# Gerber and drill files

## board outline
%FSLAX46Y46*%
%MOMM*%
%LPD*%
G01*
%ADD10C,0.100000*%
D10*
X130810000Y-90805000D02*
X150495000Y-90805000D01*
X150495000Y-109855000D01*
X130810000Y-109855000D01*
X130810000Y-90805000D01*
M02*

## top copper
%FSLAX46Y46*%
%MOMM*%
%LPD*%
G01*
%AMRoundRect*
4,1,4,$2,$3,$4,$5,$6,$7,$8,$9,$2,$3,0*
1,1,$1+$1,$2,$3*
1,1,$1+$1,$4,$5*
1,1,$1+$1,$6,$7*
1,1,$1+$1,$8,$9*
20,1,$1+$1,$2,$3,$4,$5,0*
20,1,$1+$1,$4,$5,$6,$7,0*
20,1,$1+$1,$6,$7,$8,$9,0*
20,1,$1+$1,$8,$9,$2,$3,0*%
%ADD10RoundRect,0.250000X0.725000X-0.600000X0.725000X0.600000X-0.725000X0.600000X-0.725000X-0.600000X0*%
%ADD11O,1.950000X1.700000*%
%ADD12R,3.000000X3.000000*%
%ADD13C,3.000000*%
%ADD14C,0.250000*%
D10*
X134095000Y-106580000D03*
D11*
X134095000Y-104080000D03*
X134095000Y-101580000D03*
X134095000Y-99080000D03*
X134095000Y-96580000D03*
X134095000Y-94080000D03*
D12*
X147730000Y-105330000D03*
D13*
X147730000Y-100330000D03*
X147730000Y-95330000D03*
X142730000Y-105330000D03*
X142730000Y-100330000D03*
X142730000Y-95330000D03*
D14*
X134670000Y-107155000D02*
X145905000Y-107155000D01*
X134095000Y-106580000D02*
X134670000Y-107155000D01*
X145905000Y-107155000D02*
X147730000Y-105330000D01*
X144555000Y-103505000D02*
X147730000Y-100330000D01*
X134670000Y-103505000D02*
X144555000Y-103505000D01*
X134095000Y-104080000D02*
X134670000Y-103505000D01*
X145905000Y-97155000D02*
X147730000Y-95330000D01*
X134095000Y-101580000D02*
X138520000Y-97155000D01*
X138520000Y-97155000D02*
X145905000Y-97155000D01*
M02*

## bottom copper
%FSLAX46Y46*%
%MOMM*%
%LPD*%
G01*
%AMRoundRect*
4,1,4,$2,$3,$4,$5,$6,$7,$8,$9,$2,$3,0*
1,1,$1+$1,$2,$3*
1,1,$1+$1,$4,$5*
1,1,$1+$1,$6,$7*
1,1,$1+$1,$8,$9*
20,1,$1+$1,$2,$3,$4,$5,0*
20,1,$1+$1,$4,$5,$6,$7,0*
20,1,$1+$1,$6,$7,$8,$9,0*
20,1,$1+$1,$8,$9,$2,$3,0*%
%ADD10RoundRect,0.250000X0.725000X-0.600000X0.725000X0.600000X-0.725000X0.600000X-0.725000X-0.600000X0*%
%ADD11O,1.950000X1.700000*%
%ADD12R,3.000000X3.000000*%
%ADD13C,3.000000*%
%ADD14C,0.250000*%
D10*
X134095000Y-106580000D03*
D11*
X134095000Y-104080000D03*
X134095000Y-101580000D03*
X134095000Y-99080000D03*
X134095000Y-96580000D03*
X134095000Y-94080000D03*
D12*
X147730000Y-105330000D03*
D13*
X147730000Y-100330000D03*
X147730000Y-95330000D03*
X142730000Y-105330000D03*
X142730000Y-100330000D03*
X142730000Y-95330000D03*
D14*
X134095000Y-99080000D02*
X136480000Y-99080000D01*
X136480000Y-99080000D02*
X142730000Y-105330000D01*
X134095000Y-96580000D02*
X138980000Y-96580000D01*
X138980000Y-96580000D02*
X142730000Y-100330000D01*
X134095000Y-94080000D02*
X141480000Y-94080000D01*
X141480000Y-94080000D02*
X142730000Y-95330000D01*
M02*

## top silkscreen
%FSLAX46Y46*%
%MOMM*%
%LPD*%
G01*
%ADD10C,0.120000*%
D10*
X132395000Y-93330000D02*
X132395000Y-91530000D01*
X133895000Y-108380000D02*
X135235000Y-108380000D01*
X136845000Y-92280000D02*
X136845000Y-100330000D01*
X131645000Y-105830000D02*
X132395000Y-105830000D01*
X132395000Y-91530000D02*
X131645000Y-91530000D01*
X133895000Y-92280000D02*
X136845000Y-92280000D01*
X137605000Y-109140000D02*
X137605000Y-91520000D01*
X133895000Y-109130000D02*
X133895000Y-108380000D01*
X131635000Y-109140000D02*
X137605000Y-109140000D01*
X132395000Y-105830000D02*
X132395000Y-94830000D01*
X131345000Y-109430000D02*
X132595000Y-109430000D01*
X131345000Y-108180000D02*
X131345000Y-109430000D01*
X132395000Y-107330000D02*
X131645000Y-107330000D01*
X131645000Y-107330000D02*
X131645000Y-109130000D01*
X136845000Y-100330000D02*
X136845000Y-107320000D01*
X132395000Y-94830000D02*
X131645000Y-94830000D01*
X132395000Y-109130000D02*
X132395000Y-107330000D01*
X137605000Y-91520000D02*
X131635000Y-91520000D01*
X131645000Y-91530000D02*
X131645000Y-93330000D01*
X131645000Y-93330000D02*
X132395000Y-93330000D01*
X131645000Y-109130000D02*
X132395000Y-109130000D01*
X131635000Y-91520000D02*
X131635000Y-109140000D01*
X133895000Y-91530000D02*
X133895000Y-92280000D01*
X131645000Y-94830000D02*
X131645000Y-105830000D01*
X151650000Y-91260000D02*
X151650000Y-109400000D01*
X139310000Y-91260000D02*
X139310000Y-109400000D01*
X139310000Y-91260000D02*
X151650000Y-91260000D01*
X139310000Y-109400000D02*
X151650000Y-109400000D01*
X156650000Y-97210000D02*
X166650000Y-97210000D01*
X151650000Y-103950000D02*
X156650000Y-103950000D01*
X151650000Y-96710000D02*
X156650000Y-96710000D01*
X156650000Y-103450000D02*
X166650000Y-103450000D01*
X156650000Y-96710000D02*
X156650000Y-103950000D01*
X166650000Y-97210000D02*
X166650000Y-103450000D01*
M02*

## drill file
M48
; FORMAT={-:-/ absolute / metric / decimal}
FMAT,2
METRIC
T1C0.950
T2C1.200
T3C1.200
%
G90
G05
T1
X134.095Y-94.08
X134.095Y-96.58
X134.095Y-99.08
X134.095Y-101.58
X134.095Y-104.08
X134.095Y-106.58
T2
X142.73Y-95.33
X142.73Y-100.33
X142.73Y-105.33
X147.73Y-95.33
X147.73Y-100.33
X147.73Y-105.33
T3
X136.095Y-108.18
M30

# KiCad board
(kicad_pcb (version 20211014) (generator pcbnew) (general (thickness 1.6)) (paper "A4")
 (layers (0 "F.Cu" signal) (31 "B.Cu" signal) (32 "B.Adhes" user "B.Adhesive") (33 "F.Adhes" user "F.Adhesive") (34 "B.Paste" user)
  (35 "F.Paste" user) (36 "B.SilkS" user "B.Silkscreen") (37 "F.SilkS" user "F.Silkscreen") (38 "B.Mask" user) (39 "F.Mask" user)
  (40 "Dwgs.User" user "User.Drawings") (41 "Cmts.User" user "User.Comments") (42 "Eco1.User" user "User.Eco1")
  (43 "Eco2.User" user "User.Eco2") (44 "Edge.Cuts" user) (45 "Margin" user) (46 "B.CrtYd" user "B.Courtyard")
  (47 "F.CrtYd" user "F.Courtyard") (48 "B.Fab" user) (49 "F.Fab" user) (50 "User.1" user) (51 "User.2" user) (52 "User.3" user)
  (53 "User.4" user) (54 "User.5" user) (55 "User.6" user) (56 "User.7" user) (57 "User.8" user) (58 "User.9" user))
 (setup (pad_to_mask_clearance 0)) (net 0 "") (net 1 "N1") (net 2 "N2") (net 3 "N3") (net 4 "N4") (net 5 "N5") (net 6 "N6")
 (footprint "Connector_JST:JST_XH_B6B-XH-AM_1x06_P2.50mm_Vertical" (layer "F.Cu") (at 134.095 106.58 90)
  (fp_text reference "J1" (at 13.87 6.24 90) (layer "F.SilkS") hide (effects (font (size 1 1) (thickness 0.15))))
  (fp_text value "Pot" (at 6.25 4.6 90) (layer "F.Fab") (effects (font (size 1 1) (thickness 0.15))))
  (fp_line (start 13.25 -1.7) (end 15.05 -1.7) (layer "F.SilkS") (width 0.12))
  (fp_line (start -1.8 -0.2) (end -1.8 1.14) (layer "F.SilkS") (width 0.12))
  (fp_line (start 14.3 2.75) (end 6.25 2.75) (layer "F.SilkS") (width 0.12))
  (fp_line (start 0.75 -2.45) (end 0.75 -1.7) (layer "F.SilkS") (width 0.12))
  (fp_line (start 15.05 -1.7) (end 15.05 -2.45) (layer "F.SilkS") (width 0.12))
  (fp_line (start 14.3 -0.2) (end 14.3 2.75) (layer "F.SilkS") (width 0.12))
  (fp_line (start -2.56 3.51) (end 15.06 3.51) (layer "F.SilkS") (width 0.12))
  (fp_line (start -2.55 -0.2) (end -1.8 -0.2) (layer "F.SilkS") (width 0.12))
  (fp_line (start -2.56 -2.46) (end -2.56 3.51) (layer "F.SilkS") (width 0.12))
  (fp_line (start 0.75 -1.7) (end 11.75 -1.7) (layer "F.SilkS") (width 0.12))
  (fp_line (start -2.85 -2.75) (end -2.85 -1.5) (layer "F.SilkS") (width 0.12))
  (fp_line (start -1.6 -2.75) (end -2.85 -2.75) (layer "F.SilkS") (width 0.12))
  (fp_line (start -0.75 -1.7) (end -0.75 -2.45) (layer "F.SilkS") (width 0.12))
  (fp_line (start -0.75 -2.45) (end -2.55 -2.45) (layer "F.SilkS") (width 0.12))
  (fp_line (start 6.25 2.75) (end -0.74 2.75) (layer "F.SilkS") (width 0.12))
  (fp_line (start 11.75 -1.7) (end 11.75 -2.45) (layer "F.SilkS") (width 0.12))
  (fp_line (start -2.55 -1.7) (end -0.75 -1.7) (layer "F.SilkS") (width 0.12))
  (fp_line (start 15.06 3.51) (end 15.06 -2.46) (layer "F.SilkS") (width 0.12))
  (fp_line (start 15.05 -2.45) (end 13.25 -2.45) (layer "F.SilkS") (width 0.12))
  (fp_line (start 13.25 -2.45) (end 13.25 -1.7) (layer "F.SilkS") (width 0.12))
  (fp_line (start -2.55 -2.45) (end -2.55 -1.7) (layer "F.SilkS") (width 0.12))
  (fp_line (start 15.06 -2.46) (end -2.56 -2.46) (layer "F.SilkS") (width 0.12))
  (fp_line (start 15.05 -0.2) (end 14.3 -0.2) (layer "F.SilkS") (width 0.12))
  (fp_line (start 11.75 -2.45) (end 0.75 -2.45) (layer "F.SilkS") (width 0.12))
  (pad "" np_thru_hole circle (at -1.6 2 90) (size 1.2 1.2) (drill 1.2) (layers *.Cu *.Mask))
  (pad "1" thru_hole roundrect (at 0 0 90) (size 1.7 1.95) (drill 0.95) (layers *.Cu *.Mask) (roundrect_rratio 0.147059) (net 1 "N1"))
  (pad "2" thru_hole oval (at 2.5 0 90) (size 1.7 1.95) (drill 0.95) (layers *.Cu *.Mask) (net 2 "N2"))
  (pad "3" thru_hole oval (at 5 0 90) (size 1.7 1.95) (drill 0.95) (layers *.Cu *.Mask) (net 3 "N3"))
  (pad "4" thru_hole oval (at 7.5 0 90) (size 1.7 1.95) (drill 0.95) (layers *.Cu *.Mask) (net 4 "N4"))
  (pad "5" thru_hole oval (at 10 0 90) (size 1.7 1.95) (drill 0.95) (layers *.Cu *.Mask) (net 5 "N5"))
  (pad "6" thru_hole oval (at 12.5 0 90) (size 1.7 1.95) (drill 0.95) (layers *.Cu *.Mask) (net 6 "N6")))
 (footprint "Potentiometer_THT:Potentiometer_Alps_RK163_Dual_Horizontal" (layer "F.Cu") (at 147.73 105.33 180)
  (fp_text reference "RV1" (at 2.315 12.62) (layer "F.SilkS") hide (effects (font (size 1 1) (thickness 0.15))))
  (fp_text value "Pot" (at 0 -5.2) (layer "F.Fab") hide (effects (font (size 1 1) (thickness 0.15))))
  (fp_line (start -3.92 14.07) (end -3.92 -4.07) (layer "F.SilkS") (width 0.12))
  (fp_line (start 8.42 14.07) (end 8.42 -4.07) (layer "F.SilkS") (width 0.12))
  (fp_line (start 8.42 14.07) (end -3.92 14.07) (layer "F.SilkS") (width 0.12))
  (fp_line (start 8.42 -4.07) (end -3.92 -4.07) (layer "F.SilkS") (width 0.12))
  (fp_line (start -8.92 8.12) (end -18.92 8.12) (layer "F.SilkS") (width 0.12))
  (fp_line (start -3.92 1.38) (end -8.92 1.38) (layer "F.SilkS") (width 0.12))
  (fp_line (start -3.92 8.62) (end -8.92 8.62) (layer "F.SilkS") (width 0.12))
  (fp_line (start -8.92 1.88) (end -18.92 1.88) (layer "F.SilkS") (width 0.12))
  (fp_line (start -8.92 8.62) (end -8.92 1.38) (layer "F.SilkS") (width 0.12))
  (fp_line (start -18.92 8.12) (end -18.92 1.88) (layer "F.SilkS") (width 0.12))
  (pad "1" thru_hole rect (at 0 0) (size 3 3) (drill 1.2) (layers *.Cu *.Mask) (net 1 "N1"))
  (pad "2" thru_hole circle (at 0 5) (size 3 3) (drill 1.2) (layers *.Cu *.Mask) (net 2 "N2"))
  (pad "3" thru_hole circle (at 0 10) (size 3 3) (drill 1.2) (layers *.Cu *.Mask) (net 3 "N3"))
  (pad "4" thru_hole circle (at 5 0) (size 3 3) (drill 1.2) (layers *.Cu *.Mask) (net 4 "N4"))
  (pad "5" thru_hole circle (at 5 5) (size 3 3) (drill 1.2) (layers *.Cu *.Mask) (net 5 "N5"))
  (pad "6" thru_hole circle (at 5 10) (size 3 3) (drill 1.2) (layers *.Cu *.Mask) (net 6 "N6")))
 (gr_rect (start 130.81 90.805) (end 150.495 109.855) (layer "Edge.Cuts") (width 0.1) (fill none))
 (segment (start 134.67 107.155) (end 145.905 107.155) (width 0.25) (layer "F.Cu") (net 1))
 (segment (start 134.095 106.58) (end 134.67 107.155) (width 0.25) (layer "F.Cu") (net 1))
 (segment (start 145.905 107.155) (end 147.73 105.33) (width 0.25) (layer "F.Cu") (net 1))
 (segment (start 144.555 103.505) (end 147.73 100.33) (width 0.25) (layer "F.Cu") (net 2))
 (segment (start 134.67 103.505) (end 144.555 103.505) (width 0.25) (layer "F.Cu") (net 2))
 (segment (start 134.095 104.08) (end 134.67 103.505) (width 0.25) (layer "F.Cu") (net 2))
 (segment (start 145.905 97.155) (end 147.73 95.33) (width 0.25) (layer "F.Cu") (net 3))
 (segment (start 134.095 101.58) (end 138.52 97.155) (width 0.25) (layer "F.Cu") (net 3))
 (segment (start 138.52 97.155) (end 145.905 97.155) (width 0.25) (layer "F.Cu") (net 3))
 (segment (start 134.095 99.08) (end 136.48 99.08) (width 0.25) (layer "B.Cu") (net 4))
 (segment (start 136.48 99.08) (end 142.73 105.33) (width 0.25) (layer "B.Cu") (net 4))
 (segment (start 134.095 96.58) (end 138.98 96.58) (width 0.25) (layer "B.Cu") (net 5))
 (segment (start 138.98 96.58) (end 142.73 100.33) (width 0.25) (layer "B.Cu") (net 5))
 (segment (start 134.095 94.08) (end 141.48 94.08) (width 0.25) (layer "B.Cu") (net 6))
 (segment (start 141.48 94.08) (end 142.73 95.33) (width 0.25) (layer "B.Cu") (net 6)))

